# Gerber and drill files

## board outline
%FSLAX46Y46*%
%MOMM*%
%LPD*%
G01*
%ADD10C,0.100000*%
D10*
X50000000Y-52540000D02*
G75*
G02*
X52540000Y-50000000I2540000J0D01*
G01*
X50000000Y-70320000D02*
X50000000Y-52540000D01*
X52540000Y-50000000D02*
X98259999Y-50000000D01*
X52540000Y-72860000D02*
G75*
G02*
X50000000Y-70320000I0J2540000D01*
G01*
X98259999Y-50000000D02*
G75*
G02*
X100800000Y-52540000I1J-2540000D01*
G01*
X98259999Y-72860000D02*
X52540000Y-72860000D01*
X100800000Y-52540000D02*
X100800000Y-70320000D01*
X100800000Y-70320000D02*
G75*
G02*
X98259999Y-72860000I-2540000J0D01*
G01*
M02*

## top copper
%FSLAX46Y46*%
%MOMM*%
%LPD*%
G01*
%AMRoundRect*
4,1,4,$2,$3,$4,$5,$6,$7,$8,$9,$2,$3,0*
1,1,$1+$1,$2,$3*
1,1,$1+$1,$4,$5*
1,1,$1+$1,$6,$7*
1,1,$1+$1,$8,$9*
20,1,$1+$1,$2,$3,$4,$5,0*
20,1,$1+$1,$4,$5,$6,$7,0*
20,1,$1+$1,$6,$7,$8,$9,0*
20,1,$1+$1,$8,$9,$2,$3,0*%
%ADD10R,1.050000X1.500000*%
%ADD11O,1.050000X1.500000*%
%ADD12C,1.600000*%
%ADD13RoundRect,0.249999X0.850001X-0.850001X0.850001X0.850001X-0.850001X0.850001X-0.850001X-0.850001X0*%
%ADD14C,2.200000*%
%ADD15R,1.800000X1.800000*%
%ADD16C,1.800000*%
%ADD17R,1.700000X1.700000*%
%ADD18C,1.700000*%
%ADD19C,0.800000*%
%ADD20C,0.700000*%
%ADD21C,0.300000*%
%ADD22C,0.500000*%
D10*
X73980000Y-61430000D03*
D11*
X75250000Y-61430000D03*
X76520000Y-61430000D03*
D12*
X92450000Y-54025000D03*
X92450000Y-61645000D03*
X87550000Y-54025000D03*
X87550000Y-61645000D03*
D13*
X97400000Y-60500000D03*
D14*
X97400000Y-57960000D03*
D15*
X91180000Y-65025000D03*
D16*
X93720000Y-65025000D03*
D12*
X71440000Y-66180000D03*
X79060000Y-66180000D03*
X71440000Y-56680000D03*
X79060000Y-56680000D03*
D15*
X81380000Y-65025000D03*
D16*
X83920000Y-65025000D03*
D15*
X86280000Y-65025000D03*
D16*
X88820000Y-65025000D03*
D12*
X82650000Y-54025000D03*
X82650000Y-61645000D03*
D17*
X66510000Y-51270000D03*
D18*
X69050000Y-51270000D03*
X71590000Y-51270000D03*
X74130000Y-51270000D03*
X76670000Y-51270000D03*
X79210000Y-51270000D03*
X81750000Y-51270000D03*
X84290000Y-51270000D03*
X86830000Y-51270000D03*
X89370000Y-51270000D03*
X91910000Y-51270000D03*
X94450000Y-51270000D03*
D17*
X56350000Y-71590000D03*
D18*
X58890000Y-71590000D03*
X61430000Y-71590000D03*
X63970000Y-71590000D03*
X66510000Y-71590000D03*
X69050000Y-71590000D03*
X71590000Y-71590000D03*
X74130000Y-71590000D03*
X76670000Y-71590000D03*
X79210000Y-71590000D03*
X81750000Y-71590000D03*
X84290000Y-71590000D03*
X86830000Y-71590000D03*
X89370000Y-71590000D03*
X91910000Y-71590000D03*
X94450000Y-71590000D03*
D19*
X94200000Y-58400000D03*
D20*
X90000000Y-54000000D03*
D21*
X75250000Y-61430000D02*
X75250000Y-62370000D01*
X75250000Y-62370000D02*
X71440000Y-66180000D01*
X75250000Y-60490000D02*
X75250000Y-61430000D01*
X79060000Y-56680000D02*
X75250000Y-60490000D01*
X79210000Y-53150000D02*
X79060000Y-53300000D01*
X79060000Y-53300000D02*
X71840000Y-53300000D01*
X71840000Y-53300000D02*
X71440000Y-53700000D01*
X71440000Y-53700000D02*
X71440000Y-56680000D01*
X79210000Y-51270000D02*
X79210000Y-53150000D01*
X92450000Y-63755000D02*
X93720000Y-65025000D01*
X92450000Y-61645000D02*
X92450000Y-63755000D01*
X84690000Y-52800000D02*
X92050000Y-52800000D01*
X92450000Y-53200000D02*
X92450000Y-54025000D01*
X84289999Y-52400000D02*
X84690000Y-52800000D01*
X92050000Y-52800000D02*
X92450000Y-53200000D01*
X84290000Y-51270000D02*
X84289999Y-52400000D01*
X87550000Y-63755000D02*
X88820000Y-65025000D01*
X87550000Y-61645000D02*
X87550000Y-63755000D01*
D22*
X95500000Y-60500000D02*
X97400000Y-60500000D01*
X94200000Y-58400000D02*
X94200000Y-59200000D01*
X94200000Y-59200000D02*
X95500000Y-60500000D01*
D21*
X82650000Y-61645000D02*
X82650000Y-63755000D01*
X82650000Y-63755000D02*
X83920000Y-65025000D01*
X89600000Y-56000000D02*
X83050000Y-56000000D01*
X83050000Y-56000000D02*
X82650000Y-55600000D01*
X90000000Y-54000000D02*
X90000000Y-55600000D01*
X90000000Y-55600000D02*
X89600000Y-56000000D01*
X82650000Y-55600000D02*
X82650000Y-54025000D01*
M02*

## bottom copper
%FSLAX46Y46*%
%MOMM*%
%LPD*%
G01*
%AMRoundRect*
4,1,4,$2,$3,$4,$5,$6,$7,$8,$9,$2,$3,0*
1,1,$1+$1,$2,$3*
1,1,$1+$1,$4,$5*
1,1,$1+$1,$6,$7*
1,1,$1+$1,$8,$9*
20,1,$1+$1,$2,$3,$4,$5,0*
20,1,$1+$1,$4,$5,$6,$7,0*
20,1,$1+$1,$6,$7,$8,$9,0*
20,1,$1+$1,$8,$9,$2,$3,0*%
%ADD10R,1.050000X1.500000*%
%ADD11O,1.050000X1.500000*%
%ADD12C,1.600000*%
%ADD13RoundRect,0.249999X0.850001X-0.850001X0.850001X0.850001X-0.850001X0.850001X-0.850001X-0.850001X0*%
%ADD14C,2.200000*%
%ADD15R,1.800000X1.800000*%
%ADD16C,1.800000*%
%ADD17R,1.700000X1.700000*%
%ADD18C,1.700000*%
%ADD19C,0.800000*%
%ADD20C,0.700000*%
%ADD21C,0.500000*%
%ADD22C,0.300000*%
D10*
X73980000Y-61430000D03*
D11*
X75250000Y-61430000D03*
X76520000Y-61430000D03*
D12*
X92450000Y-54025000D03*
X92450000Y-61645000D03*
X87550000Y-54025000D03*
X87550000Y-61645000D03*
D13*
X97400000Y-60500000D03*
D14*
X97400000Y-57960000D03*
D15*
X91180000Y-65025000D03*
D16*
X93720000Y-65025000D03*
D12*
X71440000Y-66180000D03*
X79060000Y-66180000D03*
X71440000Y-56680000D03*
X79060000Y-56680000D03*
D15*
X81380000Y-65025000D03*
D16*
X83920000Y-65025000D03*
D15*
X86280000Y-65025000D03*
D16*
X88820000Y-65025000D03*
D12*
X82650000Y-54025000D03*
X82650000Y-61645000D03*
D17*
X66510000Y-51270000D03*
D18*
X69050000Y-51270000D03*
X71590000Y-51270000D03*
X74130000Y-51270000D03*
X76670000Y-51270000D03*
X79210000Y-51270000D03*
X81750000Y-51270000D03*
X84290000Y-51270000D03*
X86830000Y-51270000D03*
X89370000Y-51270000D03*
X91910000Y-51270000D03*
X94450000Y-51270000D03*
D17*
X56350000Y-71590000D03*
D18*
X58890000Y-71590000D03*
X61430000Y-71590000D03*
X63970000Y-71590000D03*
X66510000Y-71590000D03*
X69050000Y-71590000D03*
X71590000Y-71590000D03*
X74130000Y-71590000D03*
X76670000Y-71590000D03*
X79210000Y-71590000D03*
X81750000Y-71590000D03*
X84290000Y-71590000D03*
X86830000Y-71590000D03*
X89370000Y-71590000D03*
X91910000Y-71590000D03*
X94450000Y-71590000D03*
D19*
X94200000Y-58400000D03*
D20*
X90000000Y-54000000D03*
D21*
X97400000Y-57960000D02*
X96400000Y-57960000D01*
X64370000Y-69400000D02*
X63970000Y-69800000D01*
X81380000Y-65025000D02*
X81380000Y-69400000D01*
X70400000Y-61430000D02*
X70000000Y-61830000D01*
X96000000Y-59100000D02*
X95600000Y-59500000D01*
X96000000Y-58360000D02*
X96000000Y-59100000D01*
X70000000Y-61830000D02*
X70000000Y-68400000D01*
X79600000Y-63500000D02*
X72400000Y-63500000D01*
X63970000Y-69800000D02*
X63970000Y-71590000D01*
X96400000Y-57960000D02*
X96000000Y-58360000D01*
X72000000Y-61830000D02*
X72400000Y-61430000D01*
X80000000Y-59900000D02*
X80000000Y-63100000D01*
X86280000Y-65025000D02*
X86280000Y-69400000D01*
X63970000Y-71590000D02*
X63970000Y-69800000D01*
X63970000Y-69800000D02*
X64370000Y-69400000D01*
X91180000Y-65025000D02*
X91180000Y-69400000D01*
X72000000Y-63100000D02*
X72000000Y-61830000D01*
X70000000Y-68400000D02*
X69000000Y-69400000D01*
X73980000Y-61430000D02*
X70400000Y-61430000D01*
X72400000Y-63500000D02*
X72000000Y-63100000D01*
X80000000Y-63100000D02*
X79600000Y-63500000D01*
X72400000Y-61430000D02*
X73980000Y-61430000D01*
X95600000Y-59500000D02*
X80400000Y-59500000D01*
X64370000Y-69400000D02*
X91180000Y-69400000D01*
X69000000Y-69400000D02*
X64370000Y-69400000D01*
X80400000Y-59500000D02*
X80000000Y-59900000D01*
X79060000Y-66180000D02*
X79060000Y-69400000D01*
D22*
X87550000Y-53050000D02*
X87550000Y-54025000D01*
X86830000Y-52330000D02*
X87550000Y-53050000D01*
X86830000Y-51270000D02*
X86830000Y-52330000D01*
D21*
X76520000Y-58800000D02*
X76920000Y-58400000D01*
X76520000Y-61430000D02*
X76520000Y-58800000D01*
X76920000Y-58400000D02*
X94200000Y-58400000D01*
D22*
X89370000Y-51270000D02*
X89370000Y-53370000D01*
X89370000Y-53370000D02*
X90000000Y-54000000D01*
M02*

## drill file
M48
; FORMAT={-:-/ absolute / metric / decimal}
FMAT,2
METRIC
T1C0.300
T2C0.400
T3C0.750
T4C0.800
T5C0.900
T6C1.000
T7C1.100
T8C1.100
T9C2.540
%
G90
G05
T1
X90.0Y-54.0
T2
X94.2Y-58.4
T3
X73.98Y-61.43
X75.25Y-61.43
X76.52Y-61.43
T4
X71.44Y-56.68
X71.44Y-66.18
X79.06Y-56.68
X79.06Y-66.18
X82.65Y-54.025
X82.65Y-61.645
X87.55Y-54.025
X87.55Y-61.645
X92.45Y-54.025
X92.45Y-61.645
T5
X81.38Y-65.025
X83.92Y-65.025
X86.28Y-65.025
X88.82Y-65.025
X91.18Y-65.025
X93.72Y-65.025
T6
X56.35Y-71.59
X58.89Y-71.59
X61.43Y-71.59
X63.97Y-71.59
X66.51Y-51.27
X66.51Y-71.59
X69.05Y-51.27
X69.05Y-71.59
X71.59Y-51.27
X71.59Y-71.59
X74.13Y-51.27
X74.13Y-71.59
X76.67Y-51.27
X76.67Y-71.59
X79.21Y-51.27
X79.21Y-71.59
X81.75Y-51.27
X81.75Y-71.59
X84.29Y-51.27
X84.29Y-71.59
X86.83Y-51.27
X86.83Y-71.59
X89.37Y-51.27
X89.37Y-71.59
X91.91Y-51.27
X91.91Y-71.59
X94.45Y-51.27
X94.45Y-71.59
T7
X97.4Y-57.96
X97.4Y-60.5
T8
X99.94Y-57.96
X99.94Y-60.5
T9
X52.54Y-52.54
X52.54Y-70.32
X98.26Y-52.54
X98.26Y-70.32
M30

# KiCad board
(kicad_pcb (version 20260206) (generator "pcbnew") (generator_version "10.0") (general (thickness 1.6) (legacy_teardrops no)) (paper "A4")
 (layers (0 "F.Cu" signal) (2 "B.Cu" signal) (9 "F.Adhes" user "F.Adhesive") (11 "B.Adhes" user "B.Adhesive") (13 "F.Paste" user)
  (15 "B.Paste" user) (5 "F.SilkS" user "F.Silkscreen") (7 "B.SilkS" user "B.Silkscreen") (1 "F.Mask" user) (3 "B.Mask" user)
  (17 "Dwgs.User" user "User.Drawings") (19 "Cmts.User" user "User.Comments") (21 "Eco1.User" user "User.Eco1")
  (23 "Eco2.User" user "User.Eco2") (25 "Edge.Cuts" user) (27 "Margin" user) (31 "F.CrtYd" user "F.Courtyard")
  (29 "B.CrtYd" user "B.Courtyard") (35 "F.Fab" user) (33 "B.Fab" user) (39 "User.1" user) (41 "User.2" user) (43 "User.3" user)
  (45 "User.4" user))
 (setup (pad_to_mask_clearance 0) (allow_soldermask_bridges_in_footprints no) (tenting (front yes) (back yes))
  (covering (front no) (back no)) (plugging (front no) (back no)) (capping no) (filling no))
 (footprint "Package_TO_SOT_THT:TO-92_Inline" (layer "F.Cu") (at 73.98 61.43)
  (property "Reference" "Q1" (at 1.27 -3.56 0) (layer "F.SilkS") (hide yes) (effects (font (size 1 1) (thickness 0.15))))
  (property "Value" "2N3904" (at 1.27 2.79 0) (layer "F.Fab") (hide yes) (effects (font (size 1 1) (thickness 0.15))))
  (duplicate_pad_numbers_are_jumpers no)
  (pad "1" thru_hole rect (at 0 0) (size 1.05 1.5) (drill 0.75) (layers "*.Cu" "*.Mask") (remove_unused_layers no) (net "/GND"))
  (pad "2" thru_hole oval (at 1.27 0) (size 1.05 1.5) (drill 0.75) (layers "*.Cu" "*.Mask") (remove_unused_layers no) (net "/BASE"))
  (pad "3" thru_hole oval (at 2.54 0) (size 1.05 1.5) (drill 0.75) (layers "*.Cu" "*.Mask") (remove_unused_layers no) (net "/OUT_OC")))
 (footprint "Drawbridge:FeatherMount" (layer "F.Cu") (at 52.54 70.32)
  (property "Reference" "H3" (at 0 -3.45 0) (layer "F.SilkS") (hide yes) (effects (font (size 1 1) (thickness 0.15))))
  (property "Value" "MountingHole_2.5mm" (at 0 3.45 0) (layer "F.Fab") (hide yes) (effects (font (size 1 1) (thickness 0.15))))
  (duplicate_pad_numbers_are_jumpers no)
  (pad "" np_thru_hole circle (at 0 0) (size 2.54 2.54) (drill 2.54) (layers "*.Cu" "*.Mask")))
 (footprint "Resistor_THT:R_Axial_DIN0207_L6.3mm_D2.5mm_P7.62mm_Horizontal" (layer "F.Cu") (at 92.45 54.025 -90)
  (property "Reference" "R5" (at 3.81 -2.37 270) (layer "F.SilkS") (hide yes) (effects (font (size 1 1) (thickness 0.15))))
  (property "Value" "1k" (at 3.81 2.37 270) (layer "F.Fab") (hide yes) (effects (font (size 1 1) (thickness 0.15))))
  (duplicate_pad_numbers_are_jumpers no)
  (pad "1" thru_hole circle (at 0 0 270) (size 1.6 1.6) (drill 0.8) (layers "*.Cu" "*.Mask") (remove_unused_layers no) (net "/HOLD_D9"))
  (pad "2" thru_hole circle (at 7.62 0 270) (size 1.6 1.6) (drill 0.8) (layers "*.Cu" "*.Mask") (remove_unused_layers no) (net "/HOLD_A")))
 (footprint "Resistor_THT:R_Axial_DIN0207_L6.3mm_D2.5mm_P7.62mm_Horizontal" (layer "F.Cu") (at 87.55 54.025 -90)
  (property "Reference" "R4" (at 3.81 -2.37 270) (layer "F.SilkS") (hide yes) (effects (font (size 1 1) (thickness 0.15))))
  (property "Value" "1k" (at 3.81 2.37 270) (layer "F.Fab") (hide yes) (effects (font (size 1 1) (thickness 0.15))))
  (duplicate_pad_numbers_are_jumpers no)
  (pad "1" thru_hole circle (at 0 0 270) (size 1.6 1.6) (drill 0.8) (layers "*.Cu" "*.Mask") (remove_unused_layers no) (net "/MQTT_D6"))
  (pad "2" thru_hole circle (at 7.62 0 270) (size 1.6 1.6) (drill 0.8) (layers "*.Cu" "*.Mask") (remove_unused_layers no) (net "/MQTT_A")))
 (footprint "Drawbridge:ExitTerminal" (layer "F.Cu") (at 97.4 60.5 90)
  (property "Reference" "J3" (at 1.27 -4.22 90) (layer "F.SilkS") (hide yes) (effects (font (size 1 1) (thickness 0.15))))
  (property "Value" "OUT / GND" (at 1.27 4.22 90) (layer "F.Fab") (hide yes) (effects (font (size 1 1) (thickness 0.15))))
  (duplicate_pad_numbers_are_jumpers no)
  (pad "" np_thru_hole circle (at 0 2.54 90) (size 1.1 1.1) (drill 1.1) (layers "*.Cu" "*.Mask"))
  (pad "" np_thru_hole circle (at 2.54 2.54 90) (size 1.1 1.1) (drill 1.1) (layers "*.Cu" "*.Mask"))
  (pad "1" thru_hole roundrect (at 0 0 90) (size 2.2 2.2) (drill 1.1) (layers "*.Cu" "*.Mask") (remove_unused_layers no)
   (roundrect_rratio 0.113636) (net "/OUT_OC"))
  (pad "2" thru_hole circle (at 2.54 0 90) (size 2.2 2.2) (drill 1.1) (layers "*.Cu" "*.Mask") (remove_unused_layers no) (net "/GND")))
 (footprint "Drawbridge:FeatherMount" (layer "F.Cu") (at 98.259999 70.32)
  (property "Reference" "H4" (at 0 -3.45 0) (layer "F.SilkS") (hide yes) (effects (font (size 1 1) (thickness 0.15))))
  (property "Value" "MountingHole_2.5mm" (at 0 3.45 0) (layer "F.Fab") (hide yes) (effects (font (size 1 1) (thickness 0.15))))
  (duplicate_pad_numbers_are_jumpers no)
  (pad "" np_thru_hole circle (at 0 0) (size 2.54 2.54) (drill 2.54) (layers "*.Cu" "*.Mask")))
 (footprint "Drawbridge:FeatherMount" (layer "F.Cu") (at 98.259999 52.54)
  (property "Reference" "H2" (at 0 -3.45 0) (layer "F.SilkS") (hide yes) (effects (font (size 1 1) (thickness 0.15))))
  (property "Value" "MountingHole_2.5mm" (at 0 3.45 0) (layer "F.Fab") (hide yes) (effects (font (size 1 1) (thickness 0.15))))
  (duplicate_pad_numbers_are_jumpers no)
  (pad "" np_thru_hole circle (at 0 0) (size 2.54 2.54) (drill 2.54) (layers "*.Cu" "*.Mask")))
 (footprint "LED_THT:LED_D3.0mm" (layer "F.Cu") (at 91.18 65.025)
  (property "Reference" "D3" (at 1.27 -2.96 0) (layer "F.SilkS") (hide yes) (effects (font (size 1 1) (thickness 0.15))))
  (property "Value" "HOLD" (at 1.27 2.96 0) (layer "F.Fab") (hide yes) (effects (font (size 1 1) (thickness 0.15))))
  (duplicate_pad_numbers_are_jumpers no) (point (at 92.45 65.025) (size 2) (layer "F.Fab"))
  (pad "1" thru_hole rect (at 0 0) (size 1.8 1.8) (drill 0.9) (layers "*.Cu" "*.Mask") (remove_unused_layers no) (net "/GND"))
  (pad "2" thru_hole circle (at 2.54 0) (size 1.8 1.8) (drill 0.9) (layers "*.Cu" "*.Mask") (remove_unused_layers no) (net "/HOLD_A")))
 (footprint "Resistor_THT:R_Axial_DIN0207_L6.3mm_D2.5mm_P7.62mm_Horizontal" (layer "F.Cu") (at 71.44 66.18)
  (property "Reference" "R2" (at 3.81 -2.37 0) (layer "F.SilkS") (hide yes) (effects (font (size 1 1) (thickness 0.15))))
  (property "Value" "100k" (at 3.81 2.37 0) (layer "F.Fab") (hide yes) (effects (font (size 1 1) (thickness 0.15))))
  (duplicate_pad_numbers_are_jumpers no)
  (pad "1" thru_hole circle (at 0 0) (size 1.6 1.6) (drill 0.8) (layers "*.Cu" "*.Mask") (remove_unused_layers no) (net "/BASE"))
  (pad "2" thru_hole circle (at 7.62 0) (size 1.6 1.6) (drill 0.8) (layers "*.Cu" "*.Mask") (remove_unused_layers no) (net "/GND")))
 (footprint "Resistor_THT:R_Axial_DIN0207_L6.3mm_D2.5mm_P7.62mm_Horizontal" (layer "F.Cu") (at 71.44 56.68)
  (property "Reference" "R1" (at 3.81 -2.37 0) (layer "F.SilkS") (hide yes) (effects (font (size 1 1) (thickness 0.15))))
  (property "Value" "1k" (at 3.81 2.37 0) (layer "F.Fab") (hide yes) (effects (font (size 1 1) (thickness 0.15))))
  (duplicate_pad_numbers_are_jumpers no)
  (pad "1" thru_hole circle (at 0 0) (size 1.6 1.6) (drill 0.8) (layers "*.Cu" "*.Mask") (remove_unused_layers no) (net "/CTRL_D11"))
  (pad "2" thru_hole circle (at 7.62 0) (size 1.6 1.6) (drill 0.8) (layers "*.Cu" "*.Mask") (remove_unused_layers no) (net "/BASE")))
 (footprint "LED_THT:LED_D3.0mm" (layer "F.Cu") (at 81.38 65.025)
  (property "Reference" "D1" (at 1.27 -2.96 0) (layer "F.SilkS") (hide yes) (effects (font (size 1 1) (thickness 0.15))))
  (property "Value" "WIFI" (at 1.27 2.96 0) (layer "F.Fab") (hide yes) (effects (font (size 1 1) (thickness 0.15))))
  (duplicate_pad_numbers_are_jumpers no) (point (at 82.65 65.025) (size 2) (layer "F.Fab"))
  (pad "1" thru_hole rect (at 0 0) (size 1.8 1.8) (drill 0.9) (layers "*.Cu" "*.Mask") (remove_unused_layers no) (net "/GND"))
  (pad "2" thru_hole circle (at 2.54 0) (size 1.8 1.8) (drill 0.9) (layers "*.Cu" "*.Mask") (remove_unused_layers no) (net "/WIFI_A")))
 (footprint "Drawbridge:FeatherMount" (layer "F.Cu") (at 52.54 52.54)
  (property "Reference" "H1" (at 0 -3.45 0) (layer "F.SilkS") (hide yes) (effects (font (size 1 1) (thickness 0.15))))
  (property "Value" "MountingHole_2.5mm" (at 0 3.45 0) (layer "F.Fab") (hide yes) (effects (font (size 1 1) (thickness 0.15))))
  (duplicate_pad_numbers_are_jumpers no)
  (pad "" np_thru_hole circle (at 0 0) (size 2.54 2.54) (drill 2.54) (layers "*.Cu" "*.Mask")))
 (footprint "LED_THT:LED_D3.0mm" (layer "F.Cu") (at 86.28 65.025)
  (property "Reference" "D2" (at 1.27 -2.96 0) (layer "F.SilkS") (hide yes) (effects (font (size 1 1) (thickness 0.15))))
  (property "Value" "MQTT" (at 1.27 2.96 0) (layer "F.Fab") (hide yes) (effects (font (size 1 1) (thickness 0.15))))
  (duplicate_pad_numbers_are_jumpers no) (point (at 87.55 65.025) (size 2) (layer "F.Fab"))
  (pad "1" thru_hole rect (at 0 0) (size 1.8 1.8) (drill 0.9) (layers "*.Cu" "*.Mask") (remove_unused_layers no) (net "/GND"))
  (pad "2" thru_hole circle (at 2.54 0) (size 1.8 1.8) (drill 0.9) (layers "*.Cu" "*.Mask") (remove_unused_layers no) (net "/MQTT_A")))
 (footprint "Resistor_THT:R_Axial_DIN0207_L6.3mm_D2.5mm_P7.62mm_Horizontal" (layer "F.Cu") (at 82.65 54.025 -90)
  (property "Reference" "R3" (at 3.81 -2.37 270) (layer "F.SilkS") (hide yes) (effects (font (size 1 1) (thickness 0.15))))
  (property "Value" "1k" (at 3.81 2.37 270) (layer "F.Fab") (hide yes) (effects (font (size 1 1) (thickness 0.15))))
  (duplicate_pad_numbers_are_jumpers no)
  (pad "1" thru_hole circle (at 0 0 270) (size 1.6 1.6) (drill 0.8) (layers "*.Cu" "*.Mask") (remove_unused_layers no) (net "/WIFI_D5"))
  (pad "2" thru_hole circle (at 7.62 0 270) (size 1.6 1.6) (drill 0.8) (layers "*.Cu" "*.Mask") (remove_unused_layers no) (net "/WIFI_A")))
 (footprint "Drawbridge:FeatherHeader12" (layer "B.Cu") (at 66.51 51.27 90)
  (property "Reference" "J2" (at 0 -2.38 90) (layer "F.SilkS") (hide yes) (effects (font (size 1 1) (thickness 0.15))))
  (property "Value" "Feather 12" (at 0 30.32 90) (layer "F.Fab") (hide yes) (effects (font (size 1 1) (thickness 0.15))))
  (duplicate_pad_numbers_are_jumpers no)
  (pad "1" thru_hole rect (at 0 0 90) (size 1.7 1.7) (drill 1) (layers "*.Cu" "*.Mask") (remove_unused_layers no)
   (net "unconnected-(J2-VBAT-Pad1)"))
  (pad "2" thru_hole circle (at 0 2.54 90) (size 1.7 1.7) (drill 1) (layers "*.Cu" "*.Mask") (remove_unused_layers no)
   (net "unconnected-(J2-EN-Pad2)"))
  (pad "3" thru_hole circle (at 0 5.08 90) (size 1.7 1.7) (drill 1) (layers "*.Cu" "*.Mask") (remove_unused_layers no)
   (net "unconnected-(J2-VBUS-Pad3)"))
  (pad "4" thru_hole circle (at 0 7.62 90) (size 1.7 1.7) (drill 1) (layers "*.Cu" "*.Mask") (remove_unused_layers no)
   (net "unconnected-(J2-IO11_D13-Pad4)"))
  (pad "5" thru_hole circle (at 0 10.16 90) (size 1.7 1.7) (drill 1) (layers "*.Cu" "*.Mask") (remove_unused_layers no)
   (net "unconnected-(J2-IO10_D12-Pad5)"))
  (pad "6" thru_hole circle (at 0 12.7 90) (size 1.7 1.7) (drill 1) (layers "*.Cu" "*.Mask") (remove_unused_layers no) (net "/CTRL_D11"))
  (pad "7" thru_hole circle (at 0 15.24 90) (size 1.7 1.7) (drill 1) (layers "*.Cu" "*.Mask") (remove_unused_layers no)
   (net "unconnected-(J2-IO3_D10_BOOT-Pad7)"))
  (pad "8" thru_hole circle (at 0 17.78 90) (size 1.7 1.7) (drill 1) (layers "*.Cu" "*.Mask") (remove_unused_layers no) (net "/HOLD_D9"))
  (pad "9" thru_hole circle (at 0 20.32 90) (size 1.7 1.7) (drill 1) (layers "*.Cu" "*.Mask") (remove_unused_layers no) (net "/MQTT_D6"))
  (pad "10" thru_hole circle (at 0 22.86 90) (size 1.7 1.7) (drill 1) (layers "*.Cu" "*.Mask") (remove_unused_layers no) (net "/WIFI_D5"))
  (pad "11" thru_hole circle (at 0 25.4 90) (size 1.7 1.7) (drill 1) (layers "*.Cu" "*.Mask") (remove_unused_layers no)
   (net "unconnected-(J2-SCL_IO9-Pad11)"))
  (pad "12" thru_hole circle (at 0 27.94 90) (size 1.7 1.7) (drill 1) (layers "*.Cu" "*.Mask") (remove_unused_layers no)
   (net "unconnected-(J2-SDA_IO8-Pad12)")))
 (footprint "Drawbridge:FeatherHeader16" (layer "B.Cu") (at 56.35 71.59 90)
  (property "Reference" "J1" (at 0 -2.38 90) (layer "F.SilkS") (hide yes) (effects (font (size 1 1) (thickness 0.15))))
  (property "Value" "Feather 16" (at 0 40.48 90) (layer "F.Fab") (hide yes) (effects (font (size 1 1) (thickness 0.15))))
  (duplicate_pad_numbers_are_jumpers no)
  (pad "1" thru_hole rect (at 0 0 90) (size 1.7 1.7) (drill 1) (layers "*.Cu" "*.Mask") (remove_unused_layers no)
   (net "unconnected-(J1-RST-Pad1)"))
  (pad "2" thru_hole circle (at 0 2.54 90) (size 1.7 1.7) (drill 1) (layers "*.Cu" "*.Mask") (remove_unused_layers no)
   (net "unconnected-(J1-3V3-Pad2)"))
  (pad "3" thru_hole circle (at 0 5.08 90) (size 1.7 1.7) (drill 1) (layers "*.Cu" "*.Mask") (remove_unused_layers no)
   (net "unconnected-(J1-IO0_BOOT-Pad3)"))
  (pad "4" thru_hole circle (at 0 7.62 90) (size 1.7 1.7) (drill 1) (layers "*.Cu" "*.Mask") (remove_unused_layers no) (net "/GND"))
  (pad "5" thru_hole circle (at 0 10.16 90) (size 1.7 1.7) (drill 1) (layers "*.Cu" "*.Mask") (remove_unused_layers no)
   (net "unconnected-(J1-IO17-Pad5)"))
  (pad "6" thru_hole circle (at 0 12.7 90) (size 1.7 1.7) (drill 1) (layers "*.Cu" "*.Mask") (remove_unused_layers no)
   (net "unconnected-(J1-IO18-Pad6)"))
  (pad "7" thru_hole circle (at 0 15.24 90) (size 1.7 1.7) (drill 1) (layers "*.Cu" "*.Mask") (remove_unused_layers no)
   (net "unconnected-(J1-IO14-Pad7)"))
  (pad "8" thru_hole circle (at 0 17.78 90) (size 1.7 1.7) (drill 1) (layers "*.Cu" "*.Mask") (remove_unused_layers no)
   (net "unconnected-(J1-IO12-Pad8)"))
  (pad "9" thru_hole circle (at 0 20.32 90) (size 1.7 1.7) (drill 1) (layers "*.Cu" "*.Mask") (remove_unused_layers no)
   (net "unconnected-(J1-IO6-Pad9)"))
  (pad "10" thru_hole circle (at 0 22.86 90) (size 1.7 1.7) (drill 1) (layers "*.Cu" "*.Mask") (remove_unused_layers no)
   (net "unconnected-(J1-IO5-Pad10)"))
  (pad "11" thru_hole circle (at 0 25.4 90) (size 1.7 1.7) (drill 1) (layers "*.Cu" "*.Mask") (remove_unused_layers no)
   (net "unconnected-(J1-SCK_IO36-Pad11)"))
  (pad "12" thru_hole circle (at 0 27.94 90) (size 1.7 1.7) (drill 1) (layers "*.Cu" "*.Mask") (remove_unused_layers no)
   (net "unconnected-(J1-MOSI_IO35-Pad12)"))
  (pad "13" thru_hole circle (at 0 30.48 90) (size 1.7 1.7) (drill 1) (layers "*.Cu" "*.Mask") (remove_unused_layers no)
   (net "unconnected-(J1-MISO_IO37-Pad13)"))
  (pad "14" thru_hole circle (at 0 33.02 90) (size 1.7 1.7) (drill 1) (layers "*.Cu" "*.Mask") (remove_unused_layers no)
   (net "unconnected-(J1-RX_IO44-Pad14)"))
  (pad "15" thru_hole circle (at 0 35.56 90) (size 1.7 1.7) (drill 1) (layers "*.Cu" "*.Mask") (remove_unused_layers no)
   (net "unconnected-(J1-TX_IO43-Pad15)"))
  (pad "16" thru_hole circle (at 0 38.1 90) (size 1.7 1.7) (drill 1) (layers "*.Cu" "*.Mask") (remove_unused_layers no)
   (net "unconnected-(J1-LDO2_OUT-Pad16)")))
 (gr_arc (start 50 52.54) (mid 50.743948 50.743948) (end 52.54 50) (stroke (width 0.1) (type default)) (layer "Edge.Cuts"))
 (gr_line (start 50 70.32) (end 50 52.54) (stroke (width 0.1) (type default)) (layer "Edge.Cuts"))
 (gr_line (start 52.54 50) (end 98.259999 50) (stroke (width 0.1) (type default)) (layer "Edge.Cuts"))
 (gr_arc (start 52.54 72.86) (mid 50.743948 72.116051) (end 50 70.32) (stroke (width 0.1) (type default)) (layer "Edge.Cuts"))
 (gr_arc (start 98.259999 50) (mid 100.056051 50.743948) (end 100.8 52.54) (stroke (width 0.1) (type default)) (layer "Edge.Cuts"))
 (gr_line (start 98.259999 72.86) (end 52.54 72.86) (stroke (width 0.1) (type default)) (layer "Edge.Cuts"))
 (gr_line (start 100.8 52.54) (end 100.8 70.32) (stroke (width 0.1) (type default)) (layer "Edge.Cuts"))
 (gr_arc (start 100.8 70.32) (mid 100.056051 72.116051) (end 98.259999 72.86) (stroke (width 0.1) (type default)) (layer "Edge.Cuts"))
 (segment (start 75.25 61.43) (end 75.25 62.37) (width 0.3) (layer "F.Cu") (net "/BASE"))
 (segment (start 75.25 62.37) (end 71.44 66.18) (width 0.3) (layer "F.Cu") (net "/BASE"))
 (segment (start 75.25 60.49) (end 75.25 61.43) (width 0.3) (layer "F.Cu") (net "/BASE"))
 (segment (start 79.06 56.68) (end 75.25 60.49) (width 0.3) (layer "F.Cu") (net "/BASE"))
 (segment (start 79.21 53.15) (end 79.06 53.3) (width 0.3) (layer "F.Cu") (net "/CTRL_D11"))
 (segment (start 79.06 53.3) (end 71.84 53.3) (width 0.3) (layer "F.Cu") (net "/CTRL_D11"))
 (segment (start 71.84 53.3) (end 71.44 53.7) (width 0.3) (layer "F.Cu") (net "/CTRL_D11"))
 (segment (start 71.44 53.7) (end 71.44 56.68) (width 0.3) (layer "F.Cu") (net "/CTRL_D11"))
 (segment (start 79.21 51.27) (end 79.21 53.15) (width 0.3) (layer "F.Cu") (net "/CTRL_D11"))
 (segment (start 97.4 57.96) (end 96.4 57.96) (width 0.5) (layer "B.Cu") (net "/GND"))
 (segment (start 64.37 69.4) (end 63.97 69.8) (width 0.5) (layer "B.Cu") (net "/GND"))
 (segment (start 81.38 65.025) (end 81.38 69.4) (width 0.5) (layer "B.Cu") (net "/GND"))
 (segment (start 70.4 61.43) (end 70 61.83) (width 0.5) (layer "B.Cu") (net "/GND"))
 (segment (start 96 59.1) (end 95.6 59.5) (width 0.5) (layer "B.Cu") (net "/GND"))
 (segment (start 96 58.36) (end 96 59.1) (width 0.5) (layer "B.Cu") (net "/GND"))
 (segment (start 70 61.83) (end 70 68.4) (width 0.5) (layer "B.Cu") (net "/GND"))
 (segment (start 79.6 63.5) (end 72.4 63.5) (width 0.5) (layer "B.Cu") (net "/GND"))
 (segment (start 63.97 69.8) (end 63.97 71.59) (width 0.5) (layer "B.Cu") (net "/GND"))
 (segment (start 96.4 57.96) (end 96 58.36) (width 0.5) (layer "B.Cu") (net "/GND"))
 (segment (start 72 61.83) (end 72.4 61.43) (width 0.5) (layer "B.Cu") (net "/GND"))
 (segment (start 80 59.9) (end 80 63.1) (width 0.5) (layer "B.Cu") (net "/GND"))
 (segment (start 86.28 65.025) (end 86.28 69.4) (width 0.5) (layer "B.Cu") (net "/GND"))
 (segment (start 63.97 71.59) (end 63.97 69.8) (width 0.5) (layer "B.Cu") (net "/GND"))
 (segment (start 63.97 69.8) (end 64.37 69.4) (width 0.5) (layer "B.Cu") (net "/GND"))
 (segment (start 91.18 65.025) (end 91.18 69.4) (width 0.5) (layer "B.Cu") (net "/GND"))
 (segment (start 72 63.1) (end 72 61.83) (width 0.5) (layer "B.Cu") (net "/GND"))
 (segment (start 70 68.4) (end 69 69.4) (width 0.5) (layer "B.Cu") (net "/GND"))
 (segment (start 73.98 61.43) (end 70.4 61.43) (width 0.5) (layer "B.Cu") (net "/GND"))
 (segment (start 72.4 63.5) (end 72 63.1) (width 0.5) (layer "B.Cu") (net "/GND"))
 (segment (start 80 63.1) (end 79.6 63.5) (width 0.5) (layer "B.Cu") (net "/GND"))
 (segment (start 72.4 61.43) (end 73.98 61.43) (width 0.5) (layer "B.Cu") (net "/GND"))
 (segment (start 95.6 59.5) (end 80.4 59.5) (width 0.5) (layer "B.Cu") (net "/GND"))
 (segment (start 64.37 69.4) (end 91.18 69.4) (width 0.5) (layer "B.Cu") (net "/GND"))
 (segment (start 69 69.4) (end 64.37 69.4) (width 0.5) (layer "B.Cu") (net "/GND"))
 (segment (start 80.4 59.5) (end 80 59.9) (width 0.5) (layer "B.Cu") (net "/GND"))
 (segment (start 79.06 66.18) (end 79.06 69.4) (width 0.5) (layer "B.Cu") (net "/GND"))
 (segment (start 92.45 63.755) (end 93.72 65.025) (width 0.3) (layer "F.Cu") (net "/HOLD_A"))
 (segment (start 92.45 61.645) (end 92.45 63.755) (width 0.3) (layer "F.Cu") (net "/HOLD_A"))
 (segment (start 84.69 52.8) (end 92.05 52.8) (width 0.3) (layer "F.Cu") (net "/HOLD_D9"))
 (segment (start 92.45 53.2) (end 92.45 54.025) (width 0.3) (layer "F.Cu") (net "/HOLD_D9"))
 (segment (start 84.289999 52.4) (end 84.69 52.8) (width 0.3) (layer "F.Cu") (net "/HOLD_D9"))
 (segment (start 92.05 52.8) (end 92.45 53.2) (width 0.3) (layer "F.Cu") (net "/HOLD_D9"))
 (segment (start 84.29 51.27) (end 84.289999 52.4) (width 0.3) (layer "F.Cu") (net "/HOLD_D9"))
 (segment (start 87.55 63.755) (end 88.82 65.025) (width 0.3) (layer "F.Cu") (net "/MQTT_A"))
 (segment (start 87.55 61.645) (end 87.55 63.755) (width 0.3) (layer "F.Cu") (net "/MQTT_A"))
 (segment (start 87.55 53.05) (end 87.55 54.025) (width 0.3) (layer "B.Cu") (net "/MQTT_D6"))
 (segment (start 86.83 52.33) (end 87.55 53.05) (width 0.3) (layer "B.Cu") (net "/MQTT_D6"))
 (segment (start 86.83 51.27) (end 86.83 52.33) (width 0.3) (layer "B.Cu") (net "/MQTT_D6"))
 (segment (start 95.5 60.5) (end 97.4 60.5) (width 0.5) (layer "F.Cu") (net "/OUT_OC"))
 (segment (start 94.2 58.4) (end 94.2 59.2) (width 0.5) (layer "F.Cu") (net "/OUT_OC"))
 (segment (start 94.2 59.2) (end 95.5 60.5) (width 0.5) (layer "F.Cu") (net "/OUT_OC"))
 (via (at 94.2 58.4) (size 0.8) (drill 0.4) (layers "F.Cu" "B.Cu") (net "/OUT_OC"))
 (segment (start 76.52 58.8) (end 76.92 58.4) (width 0.5) (layer "B.Cu") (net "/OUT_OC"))
 (segment (start 76.52 61.43) (end 76.52 58.8) (width 0.5) (layer "B.Cu") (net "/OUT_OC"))
 (segment (start 76.92 58.4) (end 94.2 58.4) (width 0.5) (layer "B.Cu") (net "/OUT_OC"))
 (segment (start 82.65 61.645) (end 82.65 63.755) (width 0.3) (layer "F.Cu") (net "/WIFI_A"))
 (segment (start 82.65 63.755) (end 83.92 65.025) (width 0.3) (layer "F.Cu") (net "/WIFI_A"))
 (segment (start 89.6 56) (end 83.05 56) (width 0.3) (layer "F.Cu") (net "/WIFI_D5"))
 (segment (start 83.05 56) (end 82.65 55.6) (width 0.3) (layer "F.Cu") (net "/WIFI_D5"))
 (segment (start 90 54) (end 90 55.6) (width 0.3) (layer "F.Cu") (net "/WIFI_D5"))
 (segment (start 90 55.6) (end 89.6 56) (width 0.3) (layer "F.Cu") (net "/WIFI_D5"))
 (segment (start 82.65 55.6) (end 82.65 54.025) (width 0.3) (layer "F.Cu") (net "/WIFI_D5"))
 (via (at 90 54) (size 0.7) (drill 0.3) (layers "F.Cu" "B.Cu") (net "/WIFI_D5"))
 (segment (start 89.37 51.27) (end 89.37 53.37) (width 0.3) (layer "B.Cu") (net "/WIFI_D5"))
 (segment (start 89.37 53.37) (end 90 54) (width 0.3) (layer "B.Cu") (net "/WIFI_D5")))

